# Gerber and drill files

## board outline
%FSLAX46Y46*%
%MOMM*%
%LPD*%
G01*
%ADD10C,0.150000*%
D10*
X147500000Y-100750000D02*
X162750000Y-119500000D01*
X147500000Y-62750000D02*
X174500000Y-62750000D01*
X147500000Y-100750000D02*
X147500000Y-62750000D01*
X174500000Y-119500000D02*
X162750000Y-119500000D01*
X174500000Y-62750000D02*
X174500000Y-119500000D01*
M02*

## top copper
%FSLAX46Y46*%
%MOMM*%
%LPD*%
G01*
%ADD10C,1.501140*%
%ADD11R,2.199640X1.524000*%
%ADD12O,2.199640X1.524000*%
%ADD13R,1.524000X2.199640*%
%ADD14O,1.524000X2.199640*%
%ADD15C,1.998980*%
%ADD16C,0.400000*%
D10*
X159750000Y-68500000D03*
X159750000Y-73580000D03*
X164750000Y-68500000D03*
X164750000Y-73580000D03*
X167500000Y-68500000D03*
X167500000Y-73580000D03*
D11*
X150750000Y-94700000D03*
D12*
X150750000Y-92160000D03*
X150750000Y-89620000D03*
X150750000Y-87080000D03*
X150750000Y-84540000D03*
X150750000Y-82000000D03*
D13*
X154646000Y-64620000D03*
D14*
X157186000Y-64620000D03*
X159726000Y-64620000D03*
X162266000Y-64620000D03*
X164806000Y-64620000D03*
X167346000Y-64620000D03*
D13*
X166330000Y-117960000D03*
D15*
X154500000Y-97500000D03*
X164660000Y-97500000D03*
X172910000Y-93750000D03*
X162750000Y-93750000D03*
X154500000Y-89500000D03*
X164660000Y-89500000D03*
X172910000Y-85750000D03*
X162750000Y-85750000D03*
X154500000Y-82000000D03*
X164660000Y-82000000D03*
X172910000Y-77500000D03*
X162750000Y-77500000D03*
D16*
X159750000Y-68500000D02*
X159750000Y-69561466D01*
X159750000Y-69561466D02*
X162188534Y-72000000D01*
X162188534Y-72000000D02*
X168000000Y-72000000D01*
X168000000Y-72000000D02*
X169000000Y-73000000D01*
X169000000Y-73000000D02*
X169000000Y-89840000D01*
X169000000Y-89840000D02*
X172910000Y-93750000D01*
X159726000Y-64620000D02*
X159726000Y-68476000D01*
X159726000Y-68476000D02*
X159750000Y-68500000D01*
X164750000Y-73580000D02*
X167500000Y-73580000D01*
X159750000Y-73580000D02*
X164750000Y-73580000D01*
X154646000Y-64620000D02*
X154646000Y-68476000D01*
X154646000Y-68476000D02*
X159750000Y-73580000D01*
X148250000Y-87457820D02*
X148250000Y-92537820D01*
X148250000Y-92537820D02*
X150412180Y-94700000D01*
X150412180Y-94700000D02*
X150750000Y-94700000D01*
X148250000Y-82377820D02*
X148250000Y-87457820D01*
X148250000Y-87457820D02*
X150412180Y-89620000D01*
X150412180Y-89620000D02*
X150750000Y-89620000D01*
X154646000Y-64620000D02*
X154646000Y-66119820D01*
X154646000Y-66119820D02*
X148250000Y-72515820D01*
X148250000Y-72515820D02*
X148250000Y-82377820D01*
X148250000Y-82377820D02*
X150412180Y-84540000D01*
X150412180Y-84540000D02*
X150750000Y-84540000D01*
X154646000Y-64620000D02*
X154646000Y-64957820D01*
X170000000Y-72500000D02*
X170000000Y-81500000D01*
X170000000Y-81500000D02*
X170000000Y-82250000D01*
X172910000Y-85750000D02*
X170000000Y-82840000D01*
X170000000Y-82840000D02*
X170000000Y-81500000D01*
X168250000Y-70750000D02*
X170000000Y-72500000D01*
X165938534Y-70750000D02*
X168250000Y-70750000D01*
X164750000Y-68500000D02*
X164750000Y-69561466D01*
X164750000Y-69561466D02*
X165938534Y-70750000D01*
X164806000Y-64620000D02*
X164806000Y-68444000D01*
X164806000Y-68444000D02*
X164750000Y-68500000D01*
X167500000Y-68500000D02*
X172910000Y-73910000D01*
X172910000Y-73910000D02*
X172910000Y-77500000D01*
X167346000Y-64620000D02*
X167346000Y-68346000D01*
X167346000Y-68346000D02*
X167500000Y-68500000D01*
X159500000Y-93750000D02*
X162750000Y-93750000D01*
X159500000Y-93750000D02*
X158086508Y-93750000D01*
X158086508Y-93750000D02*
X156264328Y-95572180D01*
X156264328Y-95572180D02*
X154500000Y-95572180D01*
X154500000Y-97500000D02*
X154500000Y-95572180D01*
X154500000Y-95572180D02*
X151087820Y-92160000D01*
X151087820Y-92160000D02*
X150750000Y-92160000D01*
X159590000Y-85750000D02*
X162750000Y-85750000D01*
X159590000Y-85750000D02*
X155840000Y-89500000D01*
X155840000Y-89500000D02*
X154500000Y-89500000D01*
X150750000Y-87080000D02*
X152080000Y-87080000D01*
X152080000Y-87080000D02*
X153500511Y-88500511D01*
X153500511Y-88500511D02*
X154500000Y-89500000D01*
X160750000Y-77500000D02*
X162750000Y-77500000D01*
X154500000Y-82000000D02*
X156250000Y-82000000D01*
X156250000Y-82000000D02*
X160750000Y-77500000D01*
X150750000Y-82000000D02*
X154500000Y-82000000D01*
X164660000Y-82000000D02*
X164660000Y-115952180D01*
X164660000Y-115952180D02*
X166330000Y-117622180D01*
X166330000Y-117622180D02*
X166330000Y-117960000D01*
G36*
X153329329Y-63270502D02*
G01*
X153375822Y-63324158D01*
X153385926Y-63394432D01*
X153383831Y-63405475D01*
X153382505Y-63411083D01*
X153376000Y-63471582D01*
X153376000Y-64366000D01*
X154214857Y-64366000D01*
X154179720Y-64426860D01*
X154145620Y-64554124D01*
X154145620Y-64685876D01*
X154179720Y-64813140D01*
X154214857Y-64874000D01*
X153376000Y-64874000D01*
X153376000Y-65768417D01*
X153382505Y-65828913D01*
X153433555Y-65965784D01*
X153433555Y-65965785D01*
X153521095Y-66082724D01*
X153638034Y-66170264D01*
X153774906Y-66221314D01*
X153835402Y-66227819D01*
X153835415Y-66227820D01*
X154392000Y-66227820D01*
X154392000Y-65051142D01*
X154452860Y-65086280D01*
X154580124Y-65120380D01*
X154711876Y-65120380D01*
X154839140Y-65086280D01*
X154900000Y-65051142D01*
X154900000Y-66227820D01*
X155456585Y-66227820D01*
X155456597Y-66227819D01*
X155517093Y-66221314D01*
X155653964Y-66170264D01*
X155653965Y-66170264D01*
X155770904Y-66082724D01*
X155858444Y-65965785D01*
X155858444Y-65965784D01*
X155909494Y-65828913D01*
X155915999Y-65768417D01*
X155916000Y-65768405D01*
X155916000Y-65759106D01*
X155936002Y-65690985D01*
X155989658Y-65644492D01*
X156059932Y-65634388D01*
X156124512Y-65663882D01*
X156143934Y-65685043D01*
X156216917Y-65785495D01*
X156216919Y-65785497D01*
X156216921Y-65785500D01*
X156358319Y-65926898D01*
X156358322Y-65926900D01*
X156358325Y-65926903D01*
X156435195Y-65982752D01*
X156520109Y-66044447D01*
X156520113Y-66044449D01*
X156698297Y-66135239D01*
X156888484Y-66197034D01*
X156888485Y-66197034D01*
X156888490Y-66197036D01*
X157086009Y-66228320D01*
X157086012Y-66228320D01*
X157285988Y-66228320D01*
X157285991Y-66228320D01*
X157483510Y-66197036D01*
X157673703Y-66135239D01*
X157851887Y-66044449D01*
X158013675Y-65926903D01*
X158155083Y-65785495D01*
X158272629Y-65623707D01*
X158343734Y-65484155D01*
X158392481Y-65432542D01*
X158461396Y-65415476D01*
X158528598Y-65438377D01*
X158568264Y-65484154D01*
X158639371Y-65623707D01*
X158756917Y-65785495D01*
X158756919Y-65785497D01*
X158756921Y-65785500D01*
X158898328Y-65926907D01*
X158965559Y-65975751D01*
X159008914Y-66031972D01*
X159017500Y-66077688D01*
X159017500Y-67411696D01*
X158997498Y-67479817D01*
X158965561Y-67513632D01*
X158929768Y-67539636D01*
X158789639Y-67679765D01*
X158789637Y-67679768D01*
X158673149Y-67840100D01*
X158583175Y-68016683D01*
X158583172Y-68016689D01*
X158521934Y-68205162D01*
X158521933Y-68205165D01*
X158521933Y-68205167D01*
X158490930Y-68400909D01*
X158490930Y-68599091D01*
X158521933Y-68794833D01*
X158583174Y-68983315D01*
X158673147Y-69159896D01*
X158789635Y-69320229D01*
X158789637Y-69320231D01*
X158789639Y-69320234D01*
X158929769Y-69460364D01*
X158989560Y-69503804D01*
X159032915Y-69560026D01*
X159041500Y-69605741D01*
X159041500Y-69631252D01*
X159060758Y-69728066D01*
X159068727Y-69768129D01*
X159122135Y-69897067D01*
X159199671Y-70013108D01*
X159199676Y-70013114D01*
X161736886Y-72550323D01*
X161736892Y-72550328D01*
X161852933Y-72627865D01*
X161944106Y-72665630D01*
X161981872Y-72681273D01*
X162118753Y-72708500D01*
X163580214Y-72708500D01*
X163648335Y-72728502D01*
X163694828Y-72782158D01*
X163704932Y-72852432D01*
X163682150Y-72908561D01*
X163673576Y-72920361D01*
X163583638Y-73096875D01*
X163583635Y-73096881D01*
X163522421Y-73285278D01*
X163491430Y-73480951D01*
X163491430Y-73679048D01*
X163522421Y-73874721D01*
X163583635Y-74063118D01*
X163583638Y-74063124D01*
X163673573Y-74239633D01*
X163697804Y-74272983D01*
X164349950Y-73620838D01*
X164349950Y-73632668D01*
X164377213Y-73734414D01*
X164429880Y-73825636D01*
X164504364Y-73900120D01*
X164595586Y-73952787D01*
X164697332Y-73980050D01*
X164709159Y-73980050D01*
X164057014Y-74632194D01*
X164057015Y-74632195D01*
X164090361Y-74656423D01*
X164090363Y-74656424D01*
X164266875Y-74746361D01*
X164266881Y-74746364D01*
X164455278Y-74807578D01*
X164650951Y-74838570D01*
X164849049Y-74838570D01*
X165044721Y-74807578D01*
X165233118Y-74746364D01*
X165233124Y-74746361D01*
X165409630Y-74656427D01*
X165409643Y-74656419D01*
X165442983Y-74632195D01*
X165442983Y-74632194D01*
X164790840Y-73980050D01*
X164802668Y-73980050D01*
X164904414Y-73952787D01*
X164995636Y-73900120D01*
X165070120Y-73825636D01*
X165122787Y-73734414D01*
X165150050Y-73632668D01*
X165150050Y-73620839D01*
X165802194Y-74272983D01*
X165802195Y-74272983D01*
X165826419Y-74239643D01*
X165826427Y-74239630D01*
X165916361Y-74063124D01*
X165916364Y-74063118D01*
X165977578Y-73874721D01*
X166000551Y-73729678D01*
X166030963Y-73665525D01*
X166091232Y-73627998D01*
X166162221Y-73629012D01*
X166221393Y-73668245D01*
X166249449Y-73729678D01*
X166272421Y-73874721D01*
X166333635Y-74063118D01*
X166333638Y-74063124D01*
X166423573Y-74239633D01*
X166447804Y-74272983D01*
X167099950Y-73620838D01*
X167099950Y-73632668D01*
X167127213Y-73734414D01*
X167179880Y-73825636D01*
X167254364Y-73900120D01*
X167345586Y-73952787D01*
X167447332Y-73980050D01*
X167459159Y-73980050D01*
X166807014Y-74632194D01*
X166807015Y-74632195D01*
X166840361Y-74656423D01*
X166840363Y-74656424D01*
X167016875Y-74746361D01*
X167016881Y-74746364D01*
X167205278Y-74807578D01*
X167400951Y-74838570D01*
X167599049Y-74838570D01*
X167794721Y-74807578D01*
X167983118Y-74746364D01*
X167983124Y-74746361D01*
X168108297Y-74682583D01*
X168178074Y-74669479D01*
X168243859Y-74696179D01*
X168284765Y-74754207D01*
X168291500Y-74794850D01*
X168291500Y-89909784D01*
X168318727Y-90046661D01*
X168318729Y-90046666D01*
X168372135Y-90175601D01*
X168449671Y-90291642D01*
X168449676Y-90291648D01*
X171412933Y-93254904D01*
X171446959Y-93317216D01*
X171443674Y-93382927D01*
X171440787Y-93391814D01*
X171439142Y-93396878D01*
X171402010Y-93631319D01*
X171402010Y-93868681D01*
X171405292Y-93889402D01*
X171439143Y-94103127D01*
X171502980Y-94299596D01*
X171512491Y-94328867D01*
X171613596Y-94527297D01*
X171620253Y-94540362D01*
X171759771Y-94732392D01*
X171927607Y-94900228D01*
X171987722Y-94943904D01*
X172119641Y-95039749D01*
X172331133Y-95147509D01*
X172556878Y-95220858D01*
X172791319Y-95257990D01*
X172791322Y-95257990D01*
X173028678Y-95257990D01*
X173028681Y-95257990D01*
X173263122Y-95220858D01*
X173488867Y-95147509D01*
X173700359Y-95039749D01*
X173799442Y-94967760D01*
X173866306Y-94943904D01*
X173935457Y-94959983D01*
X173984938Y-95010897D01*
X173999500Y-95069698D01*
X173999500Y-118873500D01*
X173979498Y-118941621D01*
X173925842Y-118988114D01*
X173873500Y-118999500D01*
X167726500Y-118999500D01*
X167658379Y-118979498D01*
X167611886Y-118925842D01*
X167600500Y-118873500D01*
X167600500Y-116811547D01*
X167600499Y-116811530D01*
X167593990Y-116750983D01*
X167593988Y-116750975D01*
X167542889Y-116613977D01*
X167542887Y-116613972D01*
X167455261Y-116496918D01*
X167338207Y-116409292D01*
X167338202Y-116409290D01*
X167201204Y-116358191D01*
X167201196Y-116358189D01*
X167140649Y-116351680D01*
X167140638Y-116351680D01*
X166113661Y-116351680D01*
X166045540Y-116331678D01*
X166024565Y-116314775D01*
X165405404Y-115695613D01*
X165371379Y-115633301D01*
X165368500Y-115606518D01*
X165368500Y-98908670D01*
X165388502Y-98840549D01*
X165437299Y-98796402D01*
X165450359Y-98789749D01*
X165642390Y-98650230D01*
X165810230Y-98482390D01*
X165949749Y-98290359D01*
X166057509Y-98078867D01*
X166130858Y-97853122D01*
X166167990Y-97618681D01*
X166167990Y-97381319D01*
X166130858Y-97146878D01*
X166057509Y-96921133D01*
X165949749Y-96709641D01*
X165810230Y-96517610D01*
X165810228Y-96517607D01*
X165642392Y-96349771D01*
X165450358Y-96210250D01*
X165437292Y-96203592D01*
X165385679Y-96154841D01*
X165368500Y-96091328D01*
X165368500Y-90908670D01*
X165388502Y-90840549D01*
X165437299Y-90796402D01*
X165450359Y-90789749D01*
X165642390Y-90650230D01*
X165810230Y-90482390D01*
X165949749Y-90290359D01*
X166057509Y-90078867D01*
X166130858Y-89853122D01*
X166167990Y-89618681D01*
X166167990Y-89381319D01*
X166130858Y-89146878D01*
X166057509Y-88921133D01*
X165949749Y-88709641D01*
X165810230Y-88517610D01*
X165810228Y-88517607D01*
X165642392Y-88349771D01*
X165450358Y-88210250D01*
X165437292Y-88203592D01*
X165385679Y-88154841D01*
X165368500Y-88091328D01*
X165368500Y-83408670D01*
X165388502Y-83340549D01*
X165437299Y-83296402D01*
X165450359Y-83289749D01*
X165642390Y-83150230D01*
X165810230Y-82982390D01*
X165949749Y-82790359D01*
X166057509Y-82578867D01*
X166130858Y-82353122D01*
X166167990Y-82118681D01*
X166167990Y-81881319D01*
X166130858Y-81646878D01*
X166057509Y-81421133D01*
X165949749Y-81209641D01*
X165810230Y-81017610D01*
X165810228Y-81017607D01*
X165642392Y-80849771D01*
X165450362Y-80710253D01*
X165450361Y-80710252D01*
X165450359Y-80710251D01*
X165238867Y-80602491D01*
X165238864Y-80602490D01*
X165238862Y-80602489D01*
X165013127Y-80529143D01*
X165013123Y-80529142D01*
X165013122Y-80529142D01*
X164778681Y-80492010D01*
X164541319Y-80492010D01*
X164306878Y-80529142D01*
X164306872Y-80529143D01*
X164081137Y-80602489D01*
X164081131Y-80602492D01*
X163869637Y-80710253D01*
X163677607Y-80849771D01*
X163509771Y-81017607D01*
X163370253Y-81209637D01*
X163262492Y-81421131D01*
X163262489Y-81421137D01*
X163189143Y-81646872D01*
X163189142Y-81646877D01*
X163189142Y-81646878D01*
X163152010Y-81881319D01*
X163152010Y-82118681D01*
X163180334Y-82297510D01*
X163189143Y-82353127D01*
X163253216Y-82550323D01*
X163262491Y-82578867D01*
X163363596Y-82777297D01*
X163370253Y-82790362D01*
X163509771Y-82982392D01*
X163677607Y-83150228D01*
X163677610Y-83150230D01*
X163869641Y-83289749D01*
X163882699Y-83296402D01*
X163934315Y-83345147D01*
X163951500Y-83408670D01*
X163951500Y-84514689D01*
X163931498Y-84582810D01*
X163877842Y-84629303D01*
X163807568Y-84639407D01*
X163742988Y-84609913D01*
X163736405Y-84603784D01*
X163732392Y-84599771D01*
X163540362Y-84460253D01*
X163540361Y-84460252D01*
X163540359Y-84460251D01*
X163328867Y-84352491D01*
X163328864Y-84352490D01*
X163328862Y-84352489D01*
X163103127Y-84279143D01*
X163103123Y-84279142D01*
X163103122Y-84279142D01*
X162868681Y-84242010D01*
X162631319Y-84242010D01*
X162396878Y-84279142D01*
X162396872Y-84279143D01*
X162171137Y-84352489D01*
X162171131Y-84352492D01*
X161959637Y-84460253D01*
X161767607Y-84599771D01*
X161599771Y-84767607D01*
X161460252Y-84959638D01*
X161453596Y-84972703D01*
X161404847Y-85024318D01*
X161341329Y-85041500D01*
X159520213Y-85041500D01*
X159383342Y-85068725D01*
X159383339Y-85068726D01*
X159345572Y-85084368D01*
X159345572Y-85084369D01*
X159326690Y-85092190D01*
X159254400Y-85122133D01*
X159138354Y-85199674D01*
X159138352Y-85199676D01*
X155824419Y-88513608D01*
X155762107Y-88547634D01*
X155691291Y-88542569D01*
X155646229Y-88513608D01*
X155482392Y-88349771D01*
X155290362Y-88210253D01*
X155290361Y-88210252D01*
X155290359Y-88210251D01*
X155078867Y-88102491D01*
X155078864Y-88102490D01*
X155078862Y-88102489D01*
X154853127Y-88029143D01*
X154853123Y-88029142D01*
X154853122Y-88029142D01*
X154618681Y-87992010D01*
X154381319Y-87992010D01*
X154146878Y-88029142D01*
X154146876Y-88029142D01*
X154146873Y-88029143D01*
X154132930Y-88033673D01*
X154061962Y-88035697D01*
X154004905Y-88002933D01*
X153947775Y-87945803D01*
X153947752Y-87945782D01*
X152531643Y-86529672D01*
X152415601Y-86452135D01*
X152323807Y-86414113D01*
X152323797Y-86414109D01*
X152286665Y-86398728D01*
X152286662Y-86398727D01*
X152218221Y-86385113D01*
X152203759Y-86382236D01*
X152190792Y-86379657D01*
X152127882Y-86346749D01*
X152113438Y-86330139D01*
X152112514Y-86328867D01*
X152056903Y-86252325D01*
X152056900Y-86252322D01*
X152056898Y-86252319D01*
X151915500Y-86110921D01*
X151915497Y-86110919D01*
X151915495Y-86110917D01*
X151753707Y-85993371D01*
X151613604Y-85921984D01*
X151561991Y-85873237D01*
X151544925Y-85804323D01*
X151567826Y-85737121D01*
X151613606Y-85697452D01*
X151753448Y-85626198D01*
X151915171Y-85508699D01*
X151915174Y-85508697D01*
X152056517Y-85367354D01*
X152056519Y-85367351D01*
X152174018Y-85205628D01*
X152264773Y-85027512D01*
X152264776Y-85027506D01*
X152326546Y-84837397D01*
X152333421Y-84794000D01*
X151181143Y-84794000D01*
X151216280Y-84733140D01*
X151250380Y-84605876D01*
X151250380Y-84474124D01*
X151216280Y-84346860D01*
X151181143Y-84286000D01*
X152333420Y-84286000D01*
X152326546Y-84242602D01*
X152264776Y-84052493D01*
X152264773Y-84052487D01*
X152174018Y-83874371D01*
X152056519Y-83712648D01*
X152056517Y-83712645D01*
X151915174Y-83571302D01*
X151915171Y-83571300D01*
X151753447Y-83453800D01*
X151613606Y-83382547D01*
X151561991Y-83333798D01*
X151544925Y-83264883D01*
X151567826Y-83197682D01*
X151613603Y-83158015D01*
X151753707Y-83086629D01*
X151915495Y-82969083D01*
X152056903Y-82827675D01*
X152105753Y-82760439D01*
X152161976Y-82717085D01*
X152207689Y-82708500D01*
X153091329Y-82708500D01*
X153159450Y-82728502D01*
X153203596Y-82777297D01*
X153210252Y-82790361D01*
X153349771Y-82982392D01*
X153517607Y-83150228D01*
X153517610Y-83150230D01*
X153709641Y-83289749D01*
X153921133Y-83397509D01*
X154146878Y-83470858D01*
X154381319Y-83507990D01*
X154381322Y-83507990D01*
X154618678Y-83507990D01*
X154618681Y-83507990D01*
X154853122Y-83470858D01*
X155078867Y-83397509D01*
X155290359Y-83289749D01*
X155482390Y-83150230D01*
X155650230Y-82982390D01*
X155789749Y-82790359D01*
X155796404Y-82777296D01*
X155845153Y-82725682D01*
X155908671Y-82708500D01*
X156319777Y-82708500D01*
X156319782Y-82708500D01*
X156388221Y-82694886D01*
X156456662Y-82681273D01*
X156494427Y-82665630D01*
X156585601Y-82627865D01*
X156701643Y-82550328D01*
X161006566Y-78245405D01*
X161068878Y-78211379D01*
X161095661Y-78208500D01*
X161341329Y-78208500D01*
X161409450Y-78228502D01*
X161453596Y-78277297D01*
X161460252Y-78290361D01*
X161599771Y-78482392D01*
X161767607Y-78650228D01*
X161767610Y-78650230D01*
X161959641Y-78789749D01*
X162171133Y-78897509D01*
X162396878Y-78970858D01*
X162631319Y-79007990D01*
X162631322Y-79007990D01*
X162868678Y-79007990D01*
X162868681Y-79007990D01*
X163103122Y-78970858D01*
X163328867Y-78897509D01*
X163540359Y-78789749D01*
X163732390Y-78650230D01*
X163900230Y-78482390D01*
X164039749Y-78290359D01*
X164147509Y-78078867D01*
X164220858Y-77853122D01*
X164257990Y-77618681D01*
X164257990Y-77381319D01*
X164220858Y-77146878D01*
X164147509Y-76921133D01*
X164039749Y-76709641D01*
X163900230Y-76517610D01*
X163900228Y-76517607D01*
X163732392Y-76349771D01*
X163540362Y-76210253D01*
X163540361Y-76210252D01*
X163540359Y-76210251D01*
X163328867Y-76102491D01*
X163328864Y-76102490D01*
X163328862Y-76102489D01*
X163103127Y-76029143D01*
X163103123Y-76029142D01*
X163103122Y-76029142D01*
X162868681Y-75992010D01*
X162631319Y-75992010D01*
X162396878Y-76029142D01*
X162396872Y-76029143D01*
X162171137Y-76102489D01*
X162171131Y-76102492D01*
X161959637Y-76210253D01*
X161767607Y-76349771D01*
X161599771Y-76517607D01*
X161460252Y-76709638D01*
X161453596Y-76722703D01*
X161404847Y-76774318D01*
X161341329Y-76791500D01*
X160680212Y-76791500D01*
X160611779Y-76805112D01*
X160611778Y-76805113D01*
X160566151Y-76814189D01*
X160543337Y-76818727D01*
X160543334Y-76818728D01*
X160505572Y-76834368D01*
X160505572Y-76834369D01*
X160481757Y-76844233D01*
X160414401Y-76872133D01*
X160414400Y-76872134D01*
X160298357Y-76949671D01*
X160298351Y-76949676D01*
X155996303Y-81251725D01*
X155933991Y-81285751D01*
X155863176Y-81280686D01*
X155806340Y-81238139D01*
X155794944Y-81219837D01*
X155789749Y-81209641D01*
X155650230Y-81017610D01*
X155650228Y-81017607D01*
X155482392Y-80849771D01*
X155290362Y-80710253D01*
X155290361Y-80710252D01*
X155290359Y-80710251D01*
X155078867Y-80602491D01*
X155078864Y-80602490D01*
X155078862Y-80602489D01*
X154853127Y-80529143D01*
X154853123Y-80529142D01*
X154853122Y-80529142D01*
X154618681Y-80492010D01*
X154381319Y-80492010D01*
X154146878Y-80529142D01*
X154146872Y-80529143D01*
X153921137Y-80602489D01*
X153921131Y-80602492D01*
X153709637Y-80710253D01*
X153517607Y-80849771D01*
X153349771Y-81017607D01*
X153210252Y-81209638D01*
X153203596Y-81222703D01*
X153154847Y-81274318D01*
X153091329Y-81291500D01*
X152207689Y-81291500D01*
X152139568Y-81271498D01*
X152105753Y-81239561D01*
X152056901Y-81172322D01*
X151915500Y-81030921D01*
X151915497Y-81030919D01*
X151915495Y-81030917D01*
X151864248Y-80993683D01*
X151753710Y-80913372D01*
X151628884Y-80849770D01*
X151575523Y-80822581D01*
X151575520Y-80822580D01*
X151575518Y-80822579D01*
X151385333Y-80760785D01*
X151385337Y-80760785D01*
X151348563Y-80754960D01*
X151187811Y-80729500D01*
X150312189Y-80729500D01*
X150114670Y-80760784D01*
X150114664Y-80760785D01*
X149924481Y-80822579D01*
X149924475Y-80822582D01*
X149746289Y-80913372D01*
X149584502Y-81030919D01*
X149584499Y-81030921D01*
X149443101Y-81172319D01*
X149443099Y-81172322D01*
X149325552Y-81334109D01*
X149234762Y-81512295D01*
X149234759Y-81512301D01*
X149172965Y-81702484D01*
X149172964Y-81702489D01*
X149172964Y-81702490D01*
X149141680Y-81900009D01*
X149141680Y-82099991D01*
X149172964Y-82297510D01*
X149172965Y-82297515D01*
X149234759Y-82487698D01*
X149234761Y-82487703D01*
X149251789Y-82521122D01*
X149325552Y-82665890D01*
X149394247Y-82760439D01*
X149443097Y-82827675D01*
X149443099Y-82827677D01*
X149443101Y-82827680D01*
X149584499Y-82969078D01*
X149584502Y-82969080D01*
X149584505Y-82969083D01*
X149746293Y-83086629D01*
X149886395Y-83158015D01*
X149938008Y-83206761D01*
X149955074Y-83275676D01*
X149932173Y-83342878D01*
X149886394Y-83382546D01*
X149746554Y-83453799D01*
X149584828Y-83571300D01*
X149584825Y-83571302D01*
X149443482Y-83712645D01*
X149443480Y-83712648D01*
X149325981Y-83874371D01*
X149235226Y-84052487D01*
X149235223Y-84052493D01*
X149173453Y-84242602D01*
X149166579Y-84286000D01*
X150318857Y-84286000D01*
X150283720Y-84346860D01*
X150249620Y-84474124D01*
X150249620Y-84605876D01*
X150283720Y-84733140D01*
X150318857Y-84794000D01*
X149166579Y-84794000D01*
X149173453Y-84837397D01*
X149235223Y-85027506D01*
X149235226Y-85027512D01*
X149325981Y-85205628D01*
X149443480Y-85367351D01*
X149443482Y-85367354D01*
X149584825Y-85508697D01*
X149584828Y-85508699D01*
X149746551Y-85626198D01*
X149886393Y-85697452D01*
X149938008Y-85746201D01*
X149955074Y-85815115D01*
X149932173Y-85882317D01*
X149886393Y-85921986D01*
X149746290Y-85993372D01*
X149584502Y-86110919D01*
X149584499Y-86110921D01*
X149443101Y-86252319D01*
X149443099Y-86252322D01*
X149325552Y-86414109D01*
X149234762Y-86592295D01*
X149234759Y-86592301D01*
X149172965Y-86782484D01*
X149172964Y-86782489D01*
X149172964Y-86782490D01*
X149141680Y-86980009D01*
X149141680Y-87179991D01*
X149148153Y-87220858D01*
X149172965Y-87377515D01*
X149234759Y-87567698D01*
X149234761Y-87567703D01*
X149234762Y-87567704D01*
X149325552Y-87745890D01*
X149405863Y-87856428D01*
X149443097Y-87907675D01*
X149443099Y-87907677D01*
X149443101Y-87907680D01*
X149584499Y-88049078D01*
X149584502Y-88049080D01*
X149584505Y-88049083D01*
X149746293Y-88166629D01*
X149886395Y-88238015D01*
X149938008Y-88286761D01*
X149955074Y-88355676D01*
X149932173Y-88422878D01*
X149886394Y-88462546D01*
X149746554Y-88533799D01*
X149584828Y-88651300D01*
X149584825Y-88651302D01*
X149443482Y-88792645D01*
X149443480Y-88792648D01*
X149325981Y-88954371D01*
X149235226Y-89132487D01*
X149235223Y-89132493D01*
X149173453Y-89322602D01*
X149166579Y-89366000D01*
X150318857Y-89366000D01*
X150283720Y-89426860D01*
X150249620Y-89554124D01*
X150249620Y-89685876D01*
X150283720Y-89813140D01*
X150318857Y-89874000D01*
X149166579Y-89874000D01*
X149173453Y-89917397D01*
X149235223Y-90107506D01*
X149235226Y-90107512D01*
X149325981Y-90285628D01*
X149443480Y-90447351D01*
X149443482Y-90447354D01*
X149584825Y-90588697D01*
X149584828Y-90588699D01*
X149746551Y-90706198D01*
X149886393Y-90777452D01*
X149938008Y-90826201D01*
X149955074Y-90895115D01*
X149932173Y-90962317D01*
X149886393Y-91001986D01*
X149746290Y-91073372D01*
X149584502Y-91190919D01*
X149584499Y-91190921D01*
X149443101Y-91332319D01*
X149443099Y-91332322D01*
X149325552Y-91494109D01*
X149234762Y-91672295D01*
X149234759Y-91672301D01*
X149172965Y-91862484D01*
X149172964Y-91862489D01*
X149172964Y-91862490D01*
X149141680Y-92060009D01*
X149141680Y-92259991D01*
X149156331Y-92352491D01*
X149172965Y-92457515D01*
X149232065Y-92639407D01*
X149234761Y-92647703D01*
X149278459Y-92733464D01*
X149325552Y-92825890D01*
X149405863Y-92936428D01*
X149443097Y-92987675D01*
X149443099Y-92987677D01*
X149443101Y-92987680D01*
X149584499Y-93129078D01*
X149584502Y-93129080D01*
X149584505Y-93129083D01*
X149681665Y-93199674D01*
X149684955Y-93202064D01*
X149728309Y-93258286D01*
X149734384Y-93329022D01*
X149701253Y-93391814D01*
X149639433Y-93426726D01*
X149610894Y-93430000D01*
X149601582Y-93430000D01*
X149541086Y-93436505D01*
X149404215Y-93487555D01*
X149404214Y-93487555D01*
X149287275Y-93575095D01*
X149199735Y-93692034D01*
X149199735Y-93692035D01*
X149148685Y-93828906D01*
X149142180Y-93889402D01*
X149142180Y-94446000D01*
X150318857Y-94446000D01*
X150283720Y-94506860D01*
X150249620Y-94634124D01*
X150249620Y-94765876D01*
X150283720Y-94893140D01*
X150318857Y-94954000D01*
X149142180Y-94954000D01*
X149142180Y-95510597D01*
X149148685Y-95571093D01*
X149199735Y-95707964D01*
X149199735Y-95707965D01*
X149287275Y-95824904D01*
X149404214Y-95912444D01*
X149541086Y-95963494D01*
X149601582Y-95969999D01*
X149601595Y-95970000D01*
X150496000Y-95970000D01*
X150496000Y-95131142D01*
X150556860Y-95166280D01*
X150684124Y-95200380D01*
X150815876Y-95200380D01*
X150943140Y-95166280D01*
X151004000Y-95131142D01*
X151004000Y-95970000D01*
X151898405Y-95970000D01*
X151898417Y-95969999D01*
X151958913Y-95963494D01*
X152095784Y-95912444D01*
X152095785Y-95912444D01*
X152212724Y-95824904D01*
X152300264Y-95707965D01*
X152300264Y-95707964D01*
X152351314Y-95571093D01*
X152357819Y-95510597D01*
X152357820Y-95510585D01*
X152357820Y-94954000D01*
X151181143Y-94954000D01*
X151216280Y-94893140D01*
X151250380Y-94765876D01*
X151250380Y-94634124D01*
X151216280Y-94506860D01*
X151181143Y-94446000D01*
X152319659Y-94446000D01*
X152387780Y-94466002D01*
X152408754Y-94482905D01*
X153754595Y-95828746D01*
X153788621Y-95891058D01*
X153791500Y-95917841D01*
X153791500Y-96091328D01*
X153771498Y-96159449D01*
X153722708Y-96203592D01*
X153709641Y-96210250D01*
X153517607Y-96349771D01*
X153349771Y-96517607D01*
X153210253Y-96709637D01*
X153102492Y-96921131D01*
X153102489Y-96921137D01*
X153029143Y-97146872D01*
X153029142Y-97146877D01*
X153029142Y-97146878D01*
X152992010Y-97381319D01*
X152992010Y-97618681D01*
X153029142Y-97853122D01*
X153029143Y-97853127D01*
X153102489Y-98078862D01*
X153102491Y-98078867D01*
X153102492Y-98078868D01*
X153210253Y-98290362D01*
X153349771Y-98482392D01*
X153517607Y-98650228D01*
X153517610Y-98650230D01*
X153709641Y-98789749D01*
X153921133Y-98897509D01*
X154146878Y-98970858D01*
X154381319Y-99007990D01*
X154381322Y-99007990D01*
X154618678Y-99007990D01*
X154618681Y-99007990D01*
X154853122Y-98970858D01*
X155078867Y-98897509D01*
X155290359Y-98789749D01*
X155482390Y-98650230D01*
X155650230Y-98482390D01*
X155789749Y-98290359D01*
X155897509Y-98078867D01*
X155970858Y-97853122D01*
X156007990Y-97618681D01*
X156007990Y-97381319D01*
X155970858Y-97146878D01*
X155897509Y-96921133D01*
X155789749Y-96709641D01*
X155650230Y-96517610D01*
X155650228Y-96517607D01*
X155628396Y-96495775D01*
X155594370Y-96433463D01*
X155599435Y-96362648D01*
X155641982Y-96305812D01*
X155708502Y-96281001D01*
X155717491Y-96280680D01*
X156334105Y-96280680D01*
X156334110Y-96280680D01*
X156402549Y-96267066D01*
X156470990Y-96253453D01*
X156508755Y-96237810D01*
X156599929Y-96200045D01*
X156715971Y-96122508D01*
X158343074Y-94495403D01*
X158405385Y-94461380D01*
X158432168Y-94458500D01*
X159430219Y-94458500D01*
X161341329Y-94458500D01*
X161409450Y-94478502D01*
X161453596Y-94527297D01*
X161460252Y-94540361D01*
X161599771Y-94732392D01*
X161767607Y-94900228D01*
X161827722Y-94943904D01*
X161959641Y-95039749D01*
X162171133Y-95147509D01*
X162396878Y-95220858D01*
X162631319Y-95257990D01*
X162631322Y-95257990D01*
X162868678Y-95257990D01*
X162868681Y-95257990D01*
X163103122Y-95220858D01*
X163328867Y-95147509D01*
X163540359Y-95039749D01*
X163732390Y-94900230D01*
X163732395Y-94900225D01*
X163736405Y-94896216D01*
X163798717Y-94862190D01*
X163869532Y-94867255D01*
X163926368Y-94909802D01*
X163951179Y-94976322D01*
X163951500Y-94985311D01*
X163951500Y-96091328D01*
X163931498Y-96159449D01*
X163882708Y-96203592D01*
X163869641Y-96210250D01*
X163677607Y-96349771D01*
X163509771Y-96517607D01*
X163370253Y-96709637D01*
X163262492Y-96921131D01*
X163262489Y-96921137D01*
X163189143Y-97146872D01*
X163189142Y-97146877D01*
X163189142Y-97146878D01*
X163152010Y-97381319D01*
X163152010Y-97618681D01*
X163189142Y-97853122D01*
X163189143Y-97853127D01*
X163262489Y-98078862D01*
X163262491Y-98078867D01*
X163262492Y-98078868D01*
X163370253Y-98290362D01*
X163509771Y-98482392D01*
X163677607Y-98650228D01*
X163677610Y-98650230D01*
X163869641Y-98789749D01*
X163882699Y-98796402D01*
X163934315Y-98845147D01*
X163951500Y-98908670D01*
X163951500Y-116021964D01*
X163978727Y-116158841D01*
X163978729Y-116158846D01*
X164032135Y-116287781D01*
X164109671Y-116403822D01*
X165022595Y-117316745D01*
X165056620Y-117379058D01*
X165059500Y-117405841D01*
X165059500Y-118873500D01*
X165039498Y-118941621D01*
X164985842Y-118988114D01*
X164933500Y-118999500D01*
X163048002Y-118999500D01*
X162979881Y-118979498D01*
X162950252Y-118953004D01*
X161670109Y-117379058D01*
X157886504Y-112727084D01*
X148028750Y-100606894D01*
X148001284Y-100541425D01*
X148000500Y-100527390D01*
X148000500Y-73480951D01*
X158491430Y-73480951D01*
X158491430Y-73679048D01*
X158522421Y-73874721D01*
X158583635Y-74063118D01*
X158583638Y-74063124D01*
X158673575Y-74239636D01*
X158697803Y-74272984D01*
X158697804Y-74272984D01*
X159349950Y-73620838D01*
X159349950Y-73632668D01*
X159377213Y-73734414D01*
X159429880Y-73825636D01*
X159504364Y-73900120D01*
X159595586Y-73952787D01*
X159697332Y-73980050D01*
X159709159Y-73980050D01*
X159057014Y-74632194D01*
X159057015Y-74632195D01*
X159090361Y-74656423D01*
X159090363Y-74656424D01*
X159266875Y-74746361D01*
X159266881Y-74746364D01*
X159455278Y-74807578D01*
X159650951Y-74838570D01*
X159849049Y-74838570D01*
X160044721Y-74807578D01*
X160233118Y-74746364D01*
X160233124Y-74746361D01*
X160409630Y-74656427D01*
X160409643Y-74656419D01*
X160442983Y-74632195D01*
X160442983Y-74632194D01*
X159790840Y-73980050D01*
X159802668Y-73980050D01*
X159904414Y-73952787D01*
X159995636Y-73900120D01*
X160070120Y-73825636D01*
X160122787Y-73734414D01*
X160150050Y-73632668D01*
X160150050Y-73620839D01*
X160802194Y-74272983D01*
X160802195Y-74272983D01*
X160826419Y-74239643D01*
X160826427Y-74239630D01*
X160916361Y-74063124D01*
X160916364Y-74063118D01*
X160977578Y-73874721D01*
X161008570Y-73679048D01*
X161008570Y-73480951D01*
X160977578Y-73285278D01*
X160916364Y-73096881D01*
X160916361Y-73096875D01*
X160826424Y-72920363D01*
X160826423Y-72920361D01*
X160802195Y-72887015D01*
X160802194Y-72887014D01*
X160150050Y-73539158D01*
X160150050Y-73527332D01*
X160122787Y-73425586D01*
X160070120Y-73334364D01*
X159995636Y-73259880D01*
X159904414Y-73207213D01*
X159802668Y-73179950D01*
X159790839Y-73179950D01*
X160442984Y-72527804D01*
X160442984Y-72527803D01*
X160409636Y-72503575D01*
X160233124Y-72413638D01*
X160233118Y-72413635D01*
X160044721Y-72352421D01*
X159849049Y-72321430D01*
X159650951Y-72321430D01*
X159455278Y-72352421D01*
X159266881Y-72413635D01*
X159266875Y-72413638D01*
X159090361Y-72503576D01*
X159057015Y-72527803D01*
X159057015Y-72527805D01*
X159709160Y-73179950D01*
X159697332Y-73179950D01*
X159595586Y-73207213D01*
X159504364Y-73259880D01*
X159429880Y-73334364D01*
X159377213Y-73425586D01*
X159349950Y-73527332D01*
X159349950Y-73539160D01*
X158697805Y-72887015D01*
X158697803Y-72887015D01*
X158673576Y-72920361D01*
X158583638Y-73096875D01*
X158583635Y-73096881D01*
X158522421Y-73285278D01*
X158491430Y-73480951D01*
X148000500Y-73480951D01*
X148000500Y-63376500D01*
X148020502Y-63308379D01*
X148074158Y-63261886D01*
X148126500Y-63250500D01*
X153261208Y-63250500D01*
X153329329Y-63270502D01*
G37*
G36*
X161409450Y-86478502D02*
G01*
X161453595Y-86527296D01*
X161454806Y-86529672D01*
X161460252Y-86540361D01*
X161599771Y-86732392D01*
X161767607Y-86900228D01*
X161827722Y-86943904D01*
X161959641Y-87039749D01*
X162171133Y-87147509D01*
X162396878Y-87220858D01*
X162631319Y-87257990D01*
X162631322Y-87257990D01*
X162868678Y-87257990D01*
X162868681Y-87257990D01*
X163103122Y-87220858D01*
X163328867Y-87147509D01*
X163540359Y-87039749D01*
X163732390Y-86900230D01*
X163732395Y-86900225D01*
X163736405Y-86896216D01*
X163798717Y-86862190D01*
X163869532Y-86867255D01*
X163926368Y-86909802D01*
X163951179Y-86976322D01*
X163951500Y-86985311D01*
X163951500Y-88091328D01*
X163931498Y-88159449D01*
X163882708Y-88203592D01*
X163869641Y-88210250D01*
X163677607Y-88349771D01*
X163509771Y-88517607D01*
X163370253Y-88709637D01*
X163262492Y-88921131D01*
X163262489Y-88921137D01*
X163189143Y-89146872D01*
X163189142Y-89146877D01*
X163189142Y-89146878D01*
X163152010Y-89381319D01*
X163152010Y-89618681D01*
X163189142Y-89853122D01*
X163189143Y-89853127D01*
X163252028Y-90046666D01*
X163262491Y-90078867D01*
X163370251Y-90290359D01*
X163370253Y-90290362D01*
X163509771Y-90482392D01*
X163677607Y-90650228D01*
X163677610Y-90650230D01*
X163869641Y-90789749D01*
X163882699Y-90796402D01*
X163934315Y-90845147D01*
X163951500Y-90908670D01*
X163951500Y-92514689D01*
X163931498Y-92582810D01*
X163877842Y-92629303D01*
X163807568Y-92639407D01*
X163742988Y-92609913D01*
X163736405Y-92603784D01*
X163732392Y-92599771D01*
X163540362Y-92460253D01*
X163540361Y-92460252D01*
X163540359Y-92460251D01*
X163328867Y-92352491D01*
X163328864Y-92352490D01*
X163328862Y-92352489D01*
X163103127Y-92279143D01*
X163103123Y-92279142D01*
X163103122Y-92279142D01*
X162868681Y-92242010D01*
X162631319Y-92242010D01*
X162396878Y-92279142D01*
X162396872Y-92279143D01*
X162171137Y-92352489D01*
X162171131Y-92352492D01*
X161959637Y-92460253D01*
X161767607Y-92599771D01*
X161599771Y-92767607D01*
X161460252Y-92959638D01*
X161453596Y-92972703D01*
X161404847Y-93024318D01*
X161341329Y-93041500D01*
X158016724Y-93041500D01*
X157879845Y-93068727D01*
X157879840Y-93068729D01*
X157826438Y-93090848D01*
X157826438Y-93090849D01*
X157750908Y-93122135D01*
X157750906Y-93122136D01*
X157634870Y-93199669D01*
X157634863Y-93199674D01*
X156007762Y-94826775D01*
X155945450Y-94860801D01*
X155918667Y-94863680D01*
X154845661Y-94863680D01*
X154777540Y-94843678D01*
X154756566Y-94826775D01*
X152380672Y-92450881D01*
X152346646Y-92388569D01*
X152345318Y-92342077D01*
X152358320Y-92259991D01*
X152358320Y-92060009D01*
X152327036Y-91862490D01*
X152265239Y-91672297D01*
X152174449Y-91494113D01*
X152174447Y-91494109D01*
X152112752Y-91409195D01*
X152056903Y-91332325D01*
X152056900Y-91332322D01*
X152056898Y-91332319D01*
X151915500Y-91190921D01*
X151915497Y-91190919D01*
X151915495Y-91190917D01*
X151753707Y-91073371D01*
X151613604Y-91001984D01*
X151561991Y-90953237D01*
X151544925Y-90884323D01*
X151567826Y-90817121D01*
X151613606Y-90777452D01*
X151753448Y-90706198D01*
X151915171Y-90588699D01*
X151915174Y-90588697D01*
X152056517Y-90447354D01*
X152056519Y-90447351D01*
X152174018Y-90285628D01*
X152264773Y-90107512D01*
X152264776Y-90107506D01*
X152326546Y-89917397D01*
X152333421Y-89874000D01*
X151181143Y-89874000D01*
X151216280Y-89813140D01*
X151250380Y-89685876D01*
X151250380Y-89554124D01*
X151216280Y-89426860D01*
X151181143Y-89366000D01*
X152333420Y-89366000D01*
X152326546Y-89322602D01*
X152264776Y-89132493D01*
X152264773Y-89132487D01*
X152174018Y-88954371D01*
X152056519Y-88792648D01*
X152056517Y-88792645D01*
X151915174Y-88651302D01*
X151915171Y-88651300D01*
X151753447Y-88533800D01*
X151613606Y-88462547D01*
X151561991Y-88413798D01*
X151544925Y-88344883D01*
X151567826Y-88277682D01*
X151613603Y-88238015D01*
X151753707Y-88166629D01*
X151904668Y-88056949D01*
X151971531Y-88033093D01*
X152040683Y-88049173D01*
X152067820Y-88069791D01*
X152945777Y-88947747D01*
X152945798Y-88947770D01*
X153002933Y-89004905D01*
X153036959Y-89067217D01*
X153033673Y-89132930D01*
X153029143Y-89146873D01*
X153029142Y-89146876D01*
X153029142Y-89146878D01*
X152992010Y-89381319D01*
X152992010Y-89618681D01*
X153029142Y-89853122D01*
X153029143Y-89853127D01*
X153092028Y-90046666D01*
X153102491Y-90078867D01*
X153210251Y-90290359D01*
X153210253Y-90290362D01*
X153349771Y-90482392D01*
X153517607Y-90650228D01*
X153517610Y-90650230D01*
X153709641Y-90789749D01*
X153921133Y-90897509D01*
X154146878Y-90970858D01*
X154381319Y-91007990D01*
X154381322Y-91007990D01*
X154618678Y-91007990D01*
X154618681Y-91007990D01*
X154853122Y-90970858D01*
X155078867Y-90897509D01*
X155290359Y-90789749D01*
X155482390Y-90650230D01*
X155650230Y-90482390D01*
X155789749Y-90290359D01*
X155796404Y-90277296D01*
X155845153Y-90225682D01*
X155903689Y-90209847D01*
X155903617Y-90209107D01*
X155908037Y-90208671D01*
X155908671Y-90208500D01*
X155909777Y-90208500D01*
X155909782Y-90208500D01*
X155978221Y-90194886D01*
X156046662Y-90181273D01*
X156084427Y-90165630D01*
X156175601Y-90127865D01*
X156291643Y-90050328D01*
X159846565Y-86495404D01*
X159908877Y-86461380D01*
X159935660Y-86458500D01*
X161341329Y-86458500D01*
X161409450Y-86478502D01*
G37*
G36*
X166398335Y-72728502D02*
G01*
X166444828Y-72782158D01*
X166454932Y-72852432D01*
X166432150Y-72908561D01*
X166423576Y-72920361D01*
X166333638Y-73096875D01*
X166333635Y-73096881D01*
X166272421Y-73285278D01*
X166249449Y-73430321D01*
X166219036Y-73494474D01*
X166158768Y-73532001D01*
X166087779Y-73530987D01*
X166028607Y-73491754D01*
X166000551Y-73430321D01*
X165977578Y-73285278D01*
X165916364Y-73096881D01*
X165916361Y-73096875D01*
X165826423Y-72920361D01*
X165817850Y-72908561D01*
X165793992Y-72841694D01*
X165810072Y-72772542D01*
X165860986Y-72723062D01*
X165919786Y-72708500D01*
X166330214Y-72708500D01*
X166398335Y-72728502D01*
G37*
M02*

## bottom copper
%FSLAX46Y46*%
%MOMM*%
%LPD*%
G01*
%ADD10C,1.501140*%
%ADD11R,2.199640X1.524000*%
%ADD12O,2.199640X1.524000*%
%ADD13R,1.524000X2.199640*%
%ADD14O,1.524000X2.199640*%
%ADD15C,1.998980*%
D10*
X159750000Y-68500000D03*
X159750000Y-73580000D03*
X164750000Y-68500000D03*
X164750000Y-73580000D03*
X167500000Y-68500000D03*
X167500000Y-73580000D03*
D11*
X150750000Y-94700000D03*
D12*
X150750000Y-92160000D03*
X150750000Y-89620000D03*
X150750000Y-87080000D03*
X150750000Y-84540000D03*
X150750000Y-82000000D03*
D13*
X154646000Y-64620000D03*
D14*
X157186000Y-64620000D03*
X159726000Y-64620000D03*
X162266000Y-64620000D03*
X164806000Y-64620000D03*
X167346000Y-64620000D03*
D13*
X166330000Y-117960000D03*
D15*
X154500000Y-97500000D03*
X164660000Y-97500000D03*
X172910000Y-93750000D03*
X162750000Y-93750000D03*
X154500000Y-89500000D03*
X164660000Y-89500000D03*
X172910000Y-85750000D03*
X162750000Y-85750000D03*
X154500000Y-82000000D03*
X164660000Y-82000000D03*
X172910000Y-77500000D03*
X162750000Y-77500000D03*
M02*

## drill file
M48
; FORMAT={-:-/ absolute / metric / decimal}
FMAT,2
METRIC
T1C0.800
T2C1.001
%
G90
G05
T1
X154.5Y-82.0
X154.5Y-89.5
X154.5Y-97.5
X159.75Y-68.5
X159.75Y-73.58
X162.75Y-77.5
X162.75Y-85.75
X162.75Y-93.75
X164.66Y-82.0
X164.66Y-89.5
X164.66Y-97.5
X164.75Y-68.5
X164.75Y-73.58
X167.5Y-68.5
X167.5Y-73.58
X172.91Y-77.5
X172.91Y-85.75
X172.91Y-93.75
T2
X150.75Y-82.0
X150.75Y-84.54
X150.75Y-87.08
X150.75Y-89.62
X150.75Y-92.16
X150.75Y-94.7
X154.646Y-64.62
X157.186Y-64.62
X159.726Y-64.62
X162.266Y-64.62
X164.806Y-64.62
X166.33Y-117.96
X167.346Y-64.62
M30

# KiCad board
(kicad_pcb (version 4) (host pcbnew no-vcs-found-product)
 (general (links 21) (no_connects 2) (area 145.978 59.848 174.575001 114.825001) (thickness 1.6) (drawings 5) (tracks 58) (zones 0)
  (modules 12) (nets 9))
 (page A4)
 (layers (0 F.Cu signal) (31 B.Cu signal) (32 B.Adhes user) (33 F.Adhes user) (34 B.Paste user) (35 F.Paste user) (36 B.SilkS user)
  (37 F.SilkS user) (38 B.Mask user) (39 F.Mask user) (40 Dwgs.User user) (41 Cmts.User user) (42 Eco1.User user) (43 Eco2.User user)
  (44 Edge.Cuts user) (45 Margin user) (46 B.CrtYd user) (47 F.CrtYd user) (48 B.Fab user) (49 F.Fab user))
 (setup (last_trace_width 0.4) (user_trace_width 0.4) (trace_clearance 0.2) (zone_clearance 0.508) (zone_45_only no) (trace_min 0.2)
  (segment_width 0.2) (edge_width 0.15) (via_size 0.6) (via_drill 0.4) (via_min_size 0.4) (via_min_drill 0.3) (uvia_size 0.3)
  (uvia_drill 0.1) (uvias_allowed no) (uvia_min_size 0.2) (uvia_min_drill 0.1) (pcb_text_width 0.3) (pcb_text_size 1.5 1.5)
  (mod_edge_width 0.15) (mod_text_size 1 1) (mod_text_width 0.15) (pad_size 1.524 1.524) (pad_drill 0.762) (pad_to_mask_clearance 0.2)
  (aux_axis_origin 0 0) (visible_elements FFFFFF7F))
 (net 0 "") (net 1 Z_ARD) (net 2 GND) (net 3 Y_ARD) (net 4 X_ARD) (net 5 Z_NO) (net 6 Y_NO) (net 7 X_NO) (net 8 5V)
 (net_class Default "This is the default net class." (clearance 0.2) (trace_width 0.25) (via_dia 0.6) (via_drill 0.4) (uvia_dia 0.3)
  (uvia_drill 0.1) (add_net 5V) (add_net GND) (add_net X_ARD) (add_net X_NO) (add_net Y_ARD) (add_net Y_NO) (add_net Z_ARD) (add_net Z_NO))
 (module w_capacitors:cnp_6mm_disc (layer F.Cu) (at 159.75 71.04 270)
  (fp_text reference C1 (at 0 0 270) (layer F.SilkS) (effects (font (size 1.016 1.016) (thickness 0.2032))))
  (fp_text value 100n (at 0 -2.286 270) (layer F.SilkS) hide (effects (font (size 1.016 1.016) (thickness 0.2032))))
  (pad 1 thru_hole circle (at -2.54 0 270) (size 1.50114 1.50114) (drill 0.8001) (layers *.Cu *.Mask F.SilkS) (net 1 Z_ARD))
  (pad 2 thru_hole circle (at 2.54 0 270) (size 1.50114 1.50114) (drill 0.8001) (layers *.Cu *.Mask F.SilkS) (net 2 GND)))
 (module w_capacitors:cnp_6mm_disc (layer F.Cu) (at 164.75 71.04 270)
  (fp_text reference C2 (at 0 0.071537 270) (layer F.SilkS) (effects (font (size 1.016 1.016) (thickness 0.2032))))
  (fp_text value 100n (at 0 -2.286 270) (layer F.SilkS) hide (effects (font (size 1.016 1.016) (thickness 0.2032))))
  (pad 1 thru_hole circle (at -2.54 0 270) (size 1.50114 1.50114) (drill 0.8001) (layers *.Cu *.Mask F.SilkS) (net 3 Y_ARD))
  (pad 2 thru_hole circle (at 2.54 0 270) (size 1.50114 1.50114) (drill 0.8001) (layers *.Cu *.Mask F.SilkS) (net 2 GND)))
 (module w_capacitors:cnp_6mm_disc (layer F.Cu) (at 167.5 71.04 270)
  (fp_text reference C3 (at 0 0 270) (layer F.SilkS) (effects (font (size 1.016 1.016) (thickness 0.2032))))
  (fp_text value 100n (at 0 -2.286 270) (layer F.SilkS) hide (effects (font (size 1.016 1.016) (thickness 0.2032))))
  (pad 1 thru_hole circle (at -2.54 0 270) (size 1.50114 1.50114) (drill 0.8001) (layers *.Cu *.Mask F.SilkS) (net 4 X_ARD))
  (pad 2 thru_hole circle (at 2.54 0 270) (size 1.50114 1.50114) (drill 0.8001) (layers *.Cu *.Mask F.SilkS) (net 2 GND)))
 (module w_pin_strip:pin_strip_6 (layer F.Cu) (at 150.75 88.35 90)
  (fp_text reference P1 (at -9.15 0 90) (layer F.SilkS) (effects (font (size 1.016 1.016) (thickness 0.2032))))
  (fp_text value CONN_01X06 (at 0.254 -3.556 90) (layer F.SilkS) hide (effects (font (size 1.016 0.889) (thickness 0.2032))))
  (pad 1 thru_hole rect (at -6.35 0 90) (size 1.524 2.19964) (drill 1.00076) (layers *.Cu *.Mask F.SilkS) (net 2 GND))
  (pad 2 thru_hole oval (at -3.81 0 90) (size 1.524 2.19964) (drill 1.00076) (layers *.Cu *.Mask F.SilkS) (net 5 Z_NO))
  (pad 3 thru_hole oval (at -1.27 0 90) (size 1.524 2.19964) (drill 1.00076) (layers *.Cu *.Mask F.SilkS) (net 2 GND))
  (pad 4 thru_hole oval (at 1.27 0 90) (size 1.524 2.19964) (drill 1.00076) (layers *.Cu *.Mask F.SilkS) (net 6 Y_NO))
  (pad 5 thru_hole oval (at 3.81 0 90) (size 1.524 2.19964) (drill 1.00076) (layers *.Cu *.Mask F.SilkS) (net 2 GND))
  (pad 6 thru_hole oval (at 6.35 0 90) (size 1.524 2.19964) (drill 1.00076) (layers *.Cu *.Mask F.SilkS) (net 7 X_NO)))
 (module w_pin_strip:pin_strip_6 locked (layer F.Cu) (at 160.996 64.62)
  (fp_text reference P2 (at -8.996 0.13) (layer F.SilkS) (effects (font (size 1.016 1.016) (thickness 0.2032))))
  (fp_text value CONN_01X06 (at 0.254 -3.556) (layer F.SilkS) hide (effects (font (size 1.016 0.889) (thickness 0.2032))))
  (pad 1 thru_hole rect (at -6.35 0) (size 1.524 2.19964) (drill 1.00076) (layers *.Cu *.Mask F.SilkS) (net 2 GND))
  (pad 2 thru_hole oval (at -3.81 0) (size 1.524 2.19964) (drill 1.00076) (layers *.Cu *.Mask F.SilkS))
  (pad 3 thru_hole oval (at -1.27 0) (size 1.524 2.19964) (drill 1.00076) (layers *.Cu *.Mask F.SilkS) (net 1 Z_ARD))
  (pad 4 thru_hole oval (at 1.27 0) (size 1.524 2.19964) (drill 1.00076) (layers *.Cu *.Mask F.SilkS))
  (pad 5 thru_hole oval (at 3.81 0) (size 1.524 2.19964) (drill 1.00076) (layers *.Cu *.Mask F.SilkS) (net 3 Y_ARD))
  (pad 6 thru_hole oval (at 6.35 0) (size 1.524 2.19964) (drill 1.00076) (layers *.Cu *.Mask F.SilkS) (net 4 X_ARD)))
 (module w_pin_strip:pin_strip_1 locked (layer F.Cu) (at 166.33 117.96)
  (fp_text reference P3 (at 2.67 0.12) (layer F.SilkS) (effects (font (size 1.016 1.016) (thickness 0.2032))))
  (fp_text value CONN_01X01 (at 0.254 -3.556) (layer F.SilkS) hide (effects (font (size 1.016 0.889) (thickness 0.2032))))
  (pad 1 thru_hole rect (at 0 0) (size 1.524 2.19964) (drill 1.00076) (layers *.Cu *.Mask F.SilkS) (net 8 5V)))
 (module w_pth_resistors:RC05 (layer F.Cu) (at 159.58 97.5) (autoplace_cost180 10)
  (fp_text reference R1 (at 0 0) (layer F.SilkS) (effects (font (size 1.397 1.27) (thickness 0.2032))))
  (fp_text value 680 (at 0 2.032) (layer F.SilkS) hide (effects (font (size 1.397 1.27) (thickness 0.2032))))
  (pad 1 thru_hole circle (at -5.08 0) (size 1.99898 1.99898) (drill 0.8001) (layers *.Cu *.Mask F.SilkS) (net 5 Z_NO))
  (pad 2 thru_hole circle (at 5.08 0) (size 1.99898 1.99898) (drill 0.8001) (layers *.Cu *.Mask F.SilkS) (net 8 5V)))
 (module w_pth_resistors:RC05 (layer F.Cu) (at 167.83 93.75 180) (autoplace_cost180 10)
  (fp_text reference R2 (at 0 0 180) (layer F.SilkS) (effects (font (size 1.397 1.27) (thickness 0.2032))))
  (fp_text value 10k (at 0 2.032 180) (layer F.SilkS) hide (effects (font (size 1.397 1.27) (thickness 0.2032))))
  (pad 1 thru_hole circle (at -5.08 0 180) (size 1.99898 1.99898) (drill 0.8001) (layers *.Cu *.Mask F.SilkS) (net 1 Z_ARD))
  (pad 2 thru_hole circle (at 5.08 0 180) (size 1.99898 1.99898) (drill 0.8001) (layers *.Cu *.Mask F.SilkS) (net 5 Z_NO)))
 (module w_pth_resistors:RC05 (layer F.Cu) (at 159.58 89.5) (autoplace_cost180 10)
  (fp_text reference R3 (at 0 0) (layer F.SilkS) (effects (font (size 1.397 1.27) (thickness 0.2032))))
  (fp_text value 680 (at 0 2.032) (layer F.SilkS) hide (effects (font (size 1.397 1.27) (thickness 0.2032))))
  (pad 1 thru_hole circle (at -5.08 0) (size 1.99898 1.99898) (drill 0.8001) (layers *.Cu *.Mask F.SilkS) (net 6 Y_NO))
  (pad 2 thru_hole circle (at 5.08 0) (size 1.99898 1.99898) (drill 0.8001) (layers *.Cu *.Mask F.SilkS) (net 8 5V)))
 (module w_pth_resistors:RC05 (layer F.Cu) (at 167.83 85.75 180) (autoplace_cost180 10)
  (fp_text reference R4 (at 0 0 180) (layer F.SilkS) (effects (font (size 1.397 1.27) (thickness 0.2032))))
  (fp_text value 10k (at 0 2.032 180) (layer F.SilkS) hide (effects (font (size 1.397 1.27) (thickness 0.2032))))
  (pad 1 thru_hole circle (at -5.08 0 180) (size 1.99898 1.99898) (drill 0.8001) (layers *.Cu *.Mask F.SilkS) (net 3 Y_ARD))
  (pad 2 thru_hole circle (at 5.08 0 180) (size 1.99898 1.99898) (drill 0.8001) (layers *.Cu *.Mask F.SilkS) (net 6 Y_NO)))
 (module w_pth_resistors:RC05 (layer F.Cu) (at 159.58 82) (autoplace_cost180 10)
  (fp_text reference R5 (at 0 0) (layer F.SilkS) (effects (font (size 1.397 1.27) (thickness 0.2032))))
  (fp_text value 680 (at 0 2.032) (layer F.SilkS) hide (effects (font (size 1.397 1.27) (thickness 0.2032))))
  (pad 1 thru_hole circle (at -5.08 0) (size 1.99898 1.99898) (drill 0.8001) (layers *.Cu *.Mask F.SilkS) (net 7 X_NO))
  (pad 2 thru_hole circle (at 5.08 0) (size 1.99898 1.99898) (drill 0.8001) (layers *.Cu *.Mask F.SilkS) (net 8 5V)))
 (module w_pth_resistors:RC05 (layer F.Cu) (at 167.83 77.5 180) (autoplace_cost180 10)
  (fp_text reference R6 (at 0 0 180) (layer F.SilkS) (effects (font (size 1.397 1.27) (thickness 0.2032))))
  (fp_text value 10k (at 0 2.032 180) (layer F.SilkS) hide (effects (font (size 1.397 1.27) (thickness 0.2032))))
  (pad 1 thru_hole circle (at -5.08 0 180) (size 1.99898 1.99898) (drill 0.8001) (layers *.Cu *.Mask F.SilkS) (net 4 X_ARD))
  (pad 2 thru_hole circle (at 5.08 0 180) (size 1.99898 1.99898) (drill 0.8001) (layers *.Cu *.Mask F.SilkS) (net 7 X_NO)))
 (gr_line (start 147.5 100.75) (end 162.75 119.5) (layer Edge.Cuts) (width 0.15))
 (gr_line (start 147.5 62.75) (end 174.5 62.75) (layer Edge.Cuts) (width 0.15))
 (gr_line (start 147.5 100.75) (end 147.5 62.75) (layer Edge.Cuts) (width 0.15))
 (gr_line (start 174.5 119.5) (end 162.75 119.5) (layer Edge.Cuts) (width 0.15))
 (gr_line (start 174.5 62.75) (end 174.5 119.5) (layer Edge.Cuts) (width 0.15))
 (segment (start 159.75 68.5) (end 159.75 69.561466) (width 0.4) (layer F.Cu) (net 1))
 (segment (start 159.75 69.561466) (end 162.188534 72) (width 0.4) (layer F.Cu) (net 1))
 (segment (start 162.188534 72) (end 168 72) (width 0.4) (layer F.Cu) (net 1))
 (segment (start 168 72) (end 169 73) (width 0.4) (layer F.Cu) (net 1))
 (segment (start 169 73) (end 169 89.84) (width 0.4) (layer F.Cu) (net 1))
 (segment (start 169 89.84) (end 172.91 93.75) (width 0.4) (layer F.Cu) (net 1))
 (segment (start 159.726 64.62) (end 159.726 68.476) (width 0.4) (layer F.Cu) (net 1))
 (segment (start 159.726 68.476) (end 159.75 68.5) (width 0.4) (layer F.Cu) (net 1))
 (segment (start 164.75 73.58) (end 167.5 73.58) (width 0.4) (layer F.Cu) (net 2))
 (segment (start 159.75 73.58) (end 164.75 73.58) (width 0.4) (layer F.Cu) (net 2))
 (segment (start 154.646 64.62) (end 154.646 68.476) (width 0.4) (layer F.Cu) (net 2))
 (segment (start 154.646 68.476) (end 159.75 73.58) (width 0.4) (layer F.Cu) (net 2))
 (segment (start 148.25 87.45782) (end 148.25 92.53782) (width 0.4) (layer F.Cu) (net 2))
 (segment (start 148.25 92.53782) (end 150.41218 94.7) (width 0.4) (layer F.Cu) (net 2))
 (segment (start 150.41218 94.7) (end 150.75 94.7) (width 0.4) (layer F.Cu) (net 2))
 (segment (start 148.25 82.37782) (end 148.25 87.45782) (width 0.4) (layer F.Cu) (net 2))
 (segment (start 148.25 87.45782) (end 150.41218 89.62) (width 0.4) (layer F.Cu) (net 2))
 (segment (start 150.41218 89.62) (end 150.75 89.62) (width 0.4) (layer F.Cu) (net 2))
 (segment (start 154.646 64.62) (end 154.646 66.11982) (width 0.4) (layer F.Cu) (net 2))
 (segment (start 154.646 66.11982) (end 148.25 72.51582) (width 0.4) (layer F.Cu) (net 2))
 (segment (start 148.25 72.51582) (end 148.25 82.37782) (width 0.4) (layer F.Cu) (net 2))
 (segment (start 148.25 82.37782) (end 150.41218 84.54) (width 0.4) (layer F.Cu) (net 2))
 (segment (start 150.41218 84.54) (end 150.75 84.54) (width 0.4) (layer F.Cu) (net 2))
 (segment (start 154.646 64.62) (end 154.646 64.95782) (width 0.4) (layer F.Cu) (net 2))
 (segment (start 170 72.5) (end 170 81.5) (width 0.4) (layer F.Cu) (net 3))
 (segment (start 170 81.5) (end 170 82.25) (width 0.4) (layer F.Cu) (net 3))
 (segment (start 172.91 85.75) (end 170 82.84) (width 0.4) (layer F.Cu) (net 3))
 (segment (start 170 82.84) (end 170 81.5) (width 0.4) (layer F.Cu) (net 3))
 (segment (start 168.25 70.75) (end 170 72.5) (width 0.4) (layer F.Cu) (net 3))
 (segment (start 165.938534 70.75) (end 168.25 70.75) (width 0.4) (layer F.Cu) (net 3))
 (segment (start 164.75 68.5) (end 164.75 69.561466) (width 0.4) (layer F.Cu) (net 3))
 (segment (start 164.75 69.561466) (end 165.938534 70.75) (width 0.4) (layer F.Cu) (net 3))
 (segment (start 164.806 64.62) (end 164.806 68.444) (width 0.4) (layer F.Cu) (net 3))
 (segment (start 164.806 68.444) (end 164.75 68.5) (width 0.4) (layer F.Cu) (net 3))
 (segment (start 167.5 68.5) (end 172.91 73.91) (width 0.4) (layer F.Cu) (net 4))
 (segment (start 172.91 73.91) (end 172.91 77.5) (width 0.4) (layer F.Cu) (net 4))
 (segment (start 167.346 64.62) (end 167.346 68.346) (width 0.4) (layer F.Cu) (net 4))
 (segment (start 167.346 68.346) (end 167.5 68.5) (width 0.4) (layer F.Cu) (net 4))
 (segment (start 159.5 93.75) (end 162.75 93.75) (width 0.4) (layer F.Cu) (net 5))
 (segment (start 159.5 93.75) (end 158.086508 93.75) (width 0.4) (layer F.Cu) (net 5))
 (segment (start 158.086508 93.75) (end 156.264328 95.57218) (width 0.4) (layer F.Cu) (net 5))
 (segment (start 156.264328 95.57218) (end 154.5 95.57218) (width 0.4) (layer F.Cu) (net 5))
 (segment (start 154.5 97.5) (end 154.5 95.57218) (width 0.4) (layer F.Cu) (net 5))
 (segment (start 154.5 95.57218) (end 151.08782 92.16) (width 0.4) (layer F.Cu) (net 5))
 (segment (start 151.08782 92.16) (end 150.75 92.16) (width 0.4) (layer F.Cu) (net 5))
 (segment (start 159.59 85.75) (end 162.75 85.75) (width 0.4) (layer F.Cu) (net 6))
 (segment (start 159.59 85.75) (end 155.84 89.5) (width 0.4) (layer F.Cu) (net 6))
 (segment (start 155.84 89.5) (end 154.5 89.5) (width 0.4) (layer F.Cu) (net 6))
 (segment (start 150.75 87.08) (end 152.08 87.08) (width 0.4) (layer F.Cu) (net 6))
 (segment (start 152.08 87.08) (end 153.500511 88.500511) (width 0.4) (layer F.Cu) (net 6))
 (segment (start 153.500511 88.500511) (end 154.5 89.5) (width 0.4) (layer F.Cu) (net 6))
 (segment (start 160.75 77.5) (end 162.75 77.5) (width 0.4) (layer F.Cu) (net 7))
 (segment (start 154.5 82) (end 156.25 82) (width 0.4) (layer F.Cu) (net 7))
 (segment (start 156.25 82) (end 160.75 77.5) (width 0.4) (layer F.Cu) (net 7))
 (segment (start 150.75 82) (end 154.5 82) (width 0.4) (layer F.Cu) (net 7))
 (segment (start 164.66 82) (end 164.66 115.95218) (width 0.4) (layer F.Cu) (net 8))
 (segment (start 164.66 115.95218) (end 166.33 117.62218) (width 0.4) (layer F.Cu) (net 8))
 (segment (start 166.33 117.62218) (end 166.33 117.96) (width 0.4) (layer F.Cu) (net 8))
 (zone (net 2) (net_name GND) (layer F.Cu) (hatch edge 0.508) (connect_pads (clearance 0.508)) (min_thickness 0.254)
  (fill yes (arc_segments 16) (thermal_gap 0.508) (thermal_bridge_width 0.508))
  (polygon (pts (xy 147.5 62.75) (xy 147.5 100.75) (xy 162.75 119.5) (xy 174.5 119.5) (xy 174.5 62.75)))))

